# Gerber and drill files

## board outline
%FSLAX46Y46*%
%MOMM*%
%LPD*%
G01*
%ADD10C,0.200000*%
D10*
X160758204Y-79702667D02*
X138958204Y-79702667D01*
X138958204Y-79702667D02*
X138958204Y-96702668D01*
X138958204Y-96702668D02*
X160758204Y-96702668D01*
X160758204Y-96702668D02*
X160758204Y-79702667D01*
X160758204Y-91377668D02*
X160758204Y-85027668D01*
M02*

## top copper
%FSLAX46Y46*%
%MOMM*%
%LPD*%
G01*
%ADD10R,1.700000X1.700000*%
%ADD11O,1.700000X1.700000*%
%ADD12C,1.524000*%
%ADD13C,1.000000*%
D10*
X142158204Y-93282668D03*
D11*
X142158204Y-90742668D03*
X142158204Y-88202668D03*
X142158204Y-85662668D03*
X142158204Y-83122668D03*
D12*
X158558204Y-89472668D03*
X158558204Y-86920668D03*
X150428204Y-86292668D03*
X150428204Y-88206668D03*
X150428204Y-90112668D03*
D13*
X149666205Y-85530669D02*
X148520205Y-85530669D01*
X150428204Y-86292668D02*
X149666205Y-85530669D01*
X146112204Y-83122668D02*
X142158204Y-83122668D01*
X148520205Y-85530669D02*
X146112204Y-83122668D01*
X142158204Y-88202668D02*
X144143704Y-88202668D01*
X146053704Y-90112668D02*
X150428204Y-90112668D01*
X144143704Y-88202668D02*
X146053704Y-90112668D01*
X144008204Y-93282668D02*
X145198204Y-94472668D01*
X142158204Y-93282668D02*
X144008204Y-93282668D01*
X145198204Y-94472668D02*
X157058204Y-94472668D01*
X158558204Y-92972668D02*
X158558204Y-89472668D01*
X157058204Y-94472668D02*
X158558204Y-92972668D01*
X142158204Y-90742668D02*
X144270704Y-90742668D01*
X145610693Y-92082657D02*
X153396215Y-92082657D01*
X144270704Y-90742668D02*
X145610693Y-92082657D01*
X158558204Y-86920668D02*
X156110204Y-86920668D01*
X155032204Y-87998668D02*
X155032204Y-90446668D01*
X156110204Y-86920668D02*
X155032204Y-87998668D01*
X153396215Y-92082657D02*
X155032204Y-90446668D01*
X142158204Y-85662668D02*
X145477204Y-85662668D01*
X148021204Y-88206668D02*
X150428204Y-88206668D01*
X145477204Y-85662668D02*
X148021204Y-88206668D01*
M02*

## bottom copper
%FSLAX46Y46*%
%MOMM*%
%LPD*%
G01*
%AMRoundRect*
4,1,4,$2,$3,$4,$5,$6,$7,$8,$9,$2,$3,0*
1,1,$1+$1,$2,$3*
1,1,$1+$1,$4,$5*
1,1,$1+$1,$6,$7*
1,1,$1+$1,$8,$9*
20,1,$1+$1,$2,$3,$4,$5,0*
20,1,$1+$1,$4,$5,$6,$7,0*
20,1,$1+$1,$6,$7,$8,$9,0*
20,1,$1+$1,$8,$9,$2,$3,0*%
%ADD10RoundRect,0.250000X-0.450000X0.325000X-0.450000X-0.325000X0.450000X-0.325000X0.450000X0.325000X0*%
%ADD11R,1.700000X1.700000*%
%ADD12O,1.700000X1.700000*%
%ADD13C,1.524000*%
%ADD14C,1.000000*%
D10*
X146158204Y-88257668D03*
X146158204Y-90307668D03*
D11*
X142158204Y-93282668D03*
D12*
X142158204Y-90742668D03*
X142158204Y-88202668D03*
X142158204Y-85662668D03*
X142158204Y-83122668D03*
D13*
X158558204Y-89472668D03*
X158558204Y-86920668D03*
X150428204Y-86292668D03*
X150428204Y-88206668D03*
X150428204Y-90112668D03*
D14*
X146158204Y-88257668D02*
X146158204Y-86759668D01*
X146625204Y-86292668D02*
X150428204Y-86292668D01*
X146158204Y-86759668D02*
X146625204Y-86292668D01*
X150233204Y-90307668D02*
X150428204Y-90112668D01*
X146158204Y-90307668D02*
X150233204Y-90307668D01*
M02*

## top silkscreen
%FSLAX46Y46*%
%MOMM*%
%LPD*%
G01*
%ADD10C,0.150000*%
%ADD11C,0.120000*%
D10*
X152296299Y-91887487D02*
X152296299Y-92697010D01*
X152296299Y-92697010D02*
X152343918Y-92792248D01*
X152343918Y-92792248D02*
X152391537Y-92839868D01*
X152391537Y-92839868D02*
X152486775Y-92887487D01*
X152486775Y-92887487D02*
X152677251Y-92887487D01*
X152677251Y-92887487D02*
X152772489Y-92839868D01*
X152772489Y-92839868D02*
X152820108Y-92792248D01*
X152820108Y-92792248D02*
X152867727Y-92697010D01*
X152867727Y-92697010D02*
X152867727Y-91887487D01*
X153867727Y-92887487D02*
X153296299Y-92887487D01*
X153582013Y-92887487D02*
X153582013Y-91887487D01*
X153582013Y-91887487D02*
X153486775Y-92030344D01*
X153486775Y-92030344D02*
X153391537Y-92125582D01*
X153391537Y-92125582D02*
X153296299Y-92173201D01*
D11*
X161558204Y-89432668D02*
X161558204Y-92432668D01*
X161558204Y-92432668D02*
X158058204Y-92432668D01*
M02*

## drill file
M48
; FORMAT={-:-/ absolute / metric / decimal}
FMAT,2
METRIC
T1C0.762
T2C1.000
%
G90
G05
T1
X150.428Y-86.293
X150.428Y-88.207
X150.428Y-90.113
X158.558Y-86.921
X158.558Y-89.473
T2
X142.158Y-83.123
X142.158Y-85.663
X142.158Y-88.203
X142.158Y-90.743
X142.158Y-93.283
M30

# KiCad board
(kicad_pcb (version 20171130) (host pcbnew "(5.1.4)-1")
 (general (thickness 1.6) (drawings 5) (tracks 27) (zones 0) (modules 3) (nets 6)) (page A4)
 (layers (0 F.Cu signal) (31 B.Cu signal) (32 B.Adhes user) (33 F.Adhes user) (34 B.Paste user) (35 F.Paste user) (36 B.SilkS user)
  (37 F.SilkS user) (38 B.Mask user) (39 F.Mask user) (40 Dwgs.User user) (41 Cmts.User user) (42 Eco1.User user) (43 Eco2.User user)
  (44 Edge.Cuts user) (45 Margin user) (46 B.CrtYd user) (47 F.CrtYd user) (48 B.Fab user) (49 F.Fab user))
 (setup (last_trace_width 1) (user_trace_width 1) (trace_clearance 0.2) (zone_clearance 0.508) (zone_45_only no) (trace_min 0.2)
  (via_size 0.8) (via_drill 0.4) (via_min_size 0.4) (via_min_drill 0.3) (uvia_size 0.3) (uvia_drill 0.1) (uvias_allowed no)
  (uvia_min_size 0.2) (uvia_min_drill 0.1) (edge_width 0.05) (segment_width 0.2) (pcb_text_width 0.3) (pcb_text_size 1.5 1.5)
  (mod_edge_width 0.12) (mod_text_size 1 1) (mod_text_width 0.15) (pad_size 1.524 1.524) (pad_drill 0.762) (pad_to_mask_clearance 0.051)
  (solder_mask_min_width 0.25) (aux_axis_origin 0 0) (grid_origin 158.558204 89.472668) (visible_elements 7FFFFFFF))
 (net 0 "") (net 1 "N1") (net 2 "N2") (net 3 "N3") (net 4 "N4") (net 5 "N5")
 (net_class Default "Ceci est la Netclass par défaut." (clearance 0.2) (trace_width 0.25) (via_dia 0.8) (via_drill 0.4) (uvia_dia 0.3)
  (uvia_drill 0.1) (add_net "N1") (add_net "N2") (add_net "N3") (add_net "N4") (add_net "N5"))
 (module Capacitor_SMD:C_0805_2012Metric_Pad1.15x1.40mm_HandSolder (layer B.Cu) (at 146.158204 89.282668 270)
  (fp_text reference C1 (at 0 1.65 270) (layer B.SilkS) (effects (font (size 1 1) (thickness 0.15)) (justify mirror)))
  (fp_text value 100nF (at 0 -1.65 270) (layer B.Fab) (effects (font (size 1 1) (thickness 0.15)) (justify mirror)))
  (pad 1 smd roundrect (at -1.025 0 270) (size 1.15 1.4) (layers B.Cu B.Paste B.Mask) (roundrect_rratio 0.217391) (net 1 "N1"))
  (pad 2 smd roundrect (at 1.025 0 270) (size 1.15 1.4) (layers B.Cu B.Paste B.Mask) (roundrect_rratio 0.217391) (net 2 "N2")))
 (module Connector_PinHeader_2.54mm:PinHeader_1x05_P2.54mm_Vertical (layer B.Cu) (at 142.158204 93.282668)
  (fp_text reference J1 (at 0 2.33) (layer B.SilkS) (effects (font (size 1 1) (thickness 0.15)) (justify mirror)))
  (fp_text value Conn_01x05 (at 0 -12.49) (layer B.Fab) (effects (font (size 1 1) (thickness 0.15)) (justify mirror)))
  (pad 1 thru_hole rect (at 0 0) (size 1.7 1.7) (drill 1) (layers *.Cu *.Mask) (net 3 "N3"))
  (pad 2 thru_hole oval (at 0 -2.54) (size 1.7 1.7) (drill 1) (layers *.Cu *.Mask) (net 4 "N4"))
  (pad 3 thru_hole oval (at 0 -5.08) (size 1.7 1.7) (drill 1) (layers *.Cu *.Mask) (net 2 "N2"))
  (pad 4 thru_hole oval (at 0 -7.62) (size 1.7 1.7) (drill 1) (layers *.Cu *.Mask) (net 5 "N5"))
  (pad 5 thru_hole oval (at 0 -10.16) (size 1.7 1.7) (drill 1) (layers *.Cu *.Mask) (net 1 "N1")))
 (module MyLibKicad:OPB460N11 (layer F.Cu) (at 154.399053 88.123483)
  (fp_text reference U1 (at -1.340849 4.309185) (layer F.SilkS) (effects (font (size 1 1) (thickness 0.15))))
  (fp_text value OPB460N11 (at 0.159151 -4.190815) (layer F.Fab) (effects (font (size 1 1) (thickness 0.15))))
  (fp_line (start 7.159151 1.309185) (end 7.159151 4.309185) (layer F.SilkS) (width 0.12))
  (fp_line (start 7.159151 4.309185) (end 3.659151 4.309185) (layer F.SilkS) (width 0.12))
  (pad 1 thru_hole circle (at 4.159151 1.349185) (size 1.524 1.524) (drill 0.762) (layers *.Cu *.Mask) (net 3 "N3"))
  (pad 2 thru_hole circle (at 4.159151 -1.202815) (size 1.524 1.524) (drill 0.762) (layers *.Cu *.Mask) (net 4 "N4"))
  (pad 3 thru_hole circle (at -3.970849 -1.830815) (size 1.524 1.524) (drill 0.762) (layers *.Cu *.Mask) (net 1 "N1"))
  (pad 4 thru_hole circle (at -3.970849 0.083185) (size 1.524 1.524) (drill 0.762) (layers *.Cu *.Mask) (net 5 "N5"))
  (pad 5 thru_hole circle (at -3.970849 1.989185) (size 1.524 1.524) (drill 0.762) (layers *.Cu *.Mask) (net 2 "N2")))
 (gr_line (start 160.758204 79.702667) (end 138.958204 79.702667) (layer Edge.Cuts) (width 0.2))
 (gr_line (start 138.958204 79.702667) (end 138.958204 96.702668) (layer Edge.Cuts) (width 0.2))
 (gr_line (start 138.958204 96.702668) (end 160.758204 96.702668) (layer Edge.Cuts) (width 0.2))
 (gr_line (start 160.758204 96.702668) (end 160.758204 79.702667) (layer Edge.Cuts) (width 0.2))
 (gr_line (start 160.758204 91.377668) (end 160.758204 85.027668) (layer Edge.Cuts) (width 0.2))
 (segment (start 149.666205 85.530669) (end 148.520205 85.530669) (width 1) (layer F.Cu) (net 1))
 (segment (start 150.428204 86.292668) (end 149.666205 85.530669) (width 1) (layer F.Cu) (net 1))
 (segment (start 146.112204 83.122668) (end 142.158204 83.122668) (width 1) (layer F.Cu) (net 1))
 (segment (start 148.520205 85.530669) (end 146.112204 83.122668) (width 1) (layer F.Cu) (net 1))
 (segment (start 146.158204 88.257668) (end 146.158204 86.759668) (width 1) (layer B.Cu) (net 1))
 (segment (start 146.625204 86.292668) (end 150.428204 86.292668) (width 1) (layer B.Cu) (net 1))
 (segment (start 146.158204 86.759668) (end 146.625204 86.292668) (width 1) (layer B.Cu) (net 1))
 (segment (start 150.233204 90.307668) (end 150.428204 90.112668) (width 1) (layer B.Cu) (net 2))
 (segment (start 146.158204 90.307668) (end 150.233204 90.307668) (width 1) (layer B.Cu) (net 2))
 (segment (start 142.158204 88.202668) (end 144.143704 88.202668) (width 1) (layer F.Cu) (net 2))
 (segment (start 146.053704 90.112668) (end 150.428204 90.112668) (width 1) (layer F.Cu) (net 2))
 (segment (start 144.143704 88.202668) (end 146.053704 90.112668) (width 1) (layer F.Cu) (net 2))
 (segment (start 144.008204 93.282668) (end 145.198204 94.472668) (width 1) (layer F.Cu) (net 3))
 (segment (start 142.158204 93.282668) (end 144.008204 93.282668) (width 1) (layer F.Cu) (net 3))
 (segment (start 145.198204 94.472668) (end 157.058204 94.472668) (width 1) (layer F.Cu) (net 3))
 (segment (start 158.558204 92.972668) (end 158.558204 89.472668) (width 1) (layer F.Cu) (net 3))
 (segment (start 157.058204 94.472668) (end 158.558204 92.972668) (width 1) (layer F.Cu) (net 3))
 (segment (start 142.158204 90.742668) (end 144.270704 90.742668) (width 1) (layer F.Cu) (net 4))
 (segment (start 145.610693 92.082657) (end 153.396215 92.082657) (width 1) (layer F.Cu) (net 4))
 (segment (start 144.270704 90.742668) (end 145.610693 92.082657) (width 1) (layer F.Cu) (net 4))
 (segment (start 158.558204 86.920668) (end 156.110204 86.920668) (width 1) (layer F.Cu) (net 4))
 (segment (start 155.032204 87.998668) (end 155.032204 90.446668) (width 1) (layer F.Cu) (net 4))
 (segment (start 156.110204 86.920668) (end 155.032204 87.998668) (width 1) (layer F.Cu) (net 4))
 (segment (start 153.396215 92.082657) (end 155.032204 90.446668) (width 1) (layer F.Cu) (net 4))
 (segment (start 142.158204 85.662668) (end 145.477204 85.662668) (width 1) (layer F.Cu) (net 5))
 (segment (start 148.021204 88.206668) (end 150.428204 88.206668) (width 1) (layer F.Cu) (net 5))
 (segment (start 145.477204 85.662668) (end 148.021204 88.206668) (width 1) (layer F.Cu) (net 5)))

